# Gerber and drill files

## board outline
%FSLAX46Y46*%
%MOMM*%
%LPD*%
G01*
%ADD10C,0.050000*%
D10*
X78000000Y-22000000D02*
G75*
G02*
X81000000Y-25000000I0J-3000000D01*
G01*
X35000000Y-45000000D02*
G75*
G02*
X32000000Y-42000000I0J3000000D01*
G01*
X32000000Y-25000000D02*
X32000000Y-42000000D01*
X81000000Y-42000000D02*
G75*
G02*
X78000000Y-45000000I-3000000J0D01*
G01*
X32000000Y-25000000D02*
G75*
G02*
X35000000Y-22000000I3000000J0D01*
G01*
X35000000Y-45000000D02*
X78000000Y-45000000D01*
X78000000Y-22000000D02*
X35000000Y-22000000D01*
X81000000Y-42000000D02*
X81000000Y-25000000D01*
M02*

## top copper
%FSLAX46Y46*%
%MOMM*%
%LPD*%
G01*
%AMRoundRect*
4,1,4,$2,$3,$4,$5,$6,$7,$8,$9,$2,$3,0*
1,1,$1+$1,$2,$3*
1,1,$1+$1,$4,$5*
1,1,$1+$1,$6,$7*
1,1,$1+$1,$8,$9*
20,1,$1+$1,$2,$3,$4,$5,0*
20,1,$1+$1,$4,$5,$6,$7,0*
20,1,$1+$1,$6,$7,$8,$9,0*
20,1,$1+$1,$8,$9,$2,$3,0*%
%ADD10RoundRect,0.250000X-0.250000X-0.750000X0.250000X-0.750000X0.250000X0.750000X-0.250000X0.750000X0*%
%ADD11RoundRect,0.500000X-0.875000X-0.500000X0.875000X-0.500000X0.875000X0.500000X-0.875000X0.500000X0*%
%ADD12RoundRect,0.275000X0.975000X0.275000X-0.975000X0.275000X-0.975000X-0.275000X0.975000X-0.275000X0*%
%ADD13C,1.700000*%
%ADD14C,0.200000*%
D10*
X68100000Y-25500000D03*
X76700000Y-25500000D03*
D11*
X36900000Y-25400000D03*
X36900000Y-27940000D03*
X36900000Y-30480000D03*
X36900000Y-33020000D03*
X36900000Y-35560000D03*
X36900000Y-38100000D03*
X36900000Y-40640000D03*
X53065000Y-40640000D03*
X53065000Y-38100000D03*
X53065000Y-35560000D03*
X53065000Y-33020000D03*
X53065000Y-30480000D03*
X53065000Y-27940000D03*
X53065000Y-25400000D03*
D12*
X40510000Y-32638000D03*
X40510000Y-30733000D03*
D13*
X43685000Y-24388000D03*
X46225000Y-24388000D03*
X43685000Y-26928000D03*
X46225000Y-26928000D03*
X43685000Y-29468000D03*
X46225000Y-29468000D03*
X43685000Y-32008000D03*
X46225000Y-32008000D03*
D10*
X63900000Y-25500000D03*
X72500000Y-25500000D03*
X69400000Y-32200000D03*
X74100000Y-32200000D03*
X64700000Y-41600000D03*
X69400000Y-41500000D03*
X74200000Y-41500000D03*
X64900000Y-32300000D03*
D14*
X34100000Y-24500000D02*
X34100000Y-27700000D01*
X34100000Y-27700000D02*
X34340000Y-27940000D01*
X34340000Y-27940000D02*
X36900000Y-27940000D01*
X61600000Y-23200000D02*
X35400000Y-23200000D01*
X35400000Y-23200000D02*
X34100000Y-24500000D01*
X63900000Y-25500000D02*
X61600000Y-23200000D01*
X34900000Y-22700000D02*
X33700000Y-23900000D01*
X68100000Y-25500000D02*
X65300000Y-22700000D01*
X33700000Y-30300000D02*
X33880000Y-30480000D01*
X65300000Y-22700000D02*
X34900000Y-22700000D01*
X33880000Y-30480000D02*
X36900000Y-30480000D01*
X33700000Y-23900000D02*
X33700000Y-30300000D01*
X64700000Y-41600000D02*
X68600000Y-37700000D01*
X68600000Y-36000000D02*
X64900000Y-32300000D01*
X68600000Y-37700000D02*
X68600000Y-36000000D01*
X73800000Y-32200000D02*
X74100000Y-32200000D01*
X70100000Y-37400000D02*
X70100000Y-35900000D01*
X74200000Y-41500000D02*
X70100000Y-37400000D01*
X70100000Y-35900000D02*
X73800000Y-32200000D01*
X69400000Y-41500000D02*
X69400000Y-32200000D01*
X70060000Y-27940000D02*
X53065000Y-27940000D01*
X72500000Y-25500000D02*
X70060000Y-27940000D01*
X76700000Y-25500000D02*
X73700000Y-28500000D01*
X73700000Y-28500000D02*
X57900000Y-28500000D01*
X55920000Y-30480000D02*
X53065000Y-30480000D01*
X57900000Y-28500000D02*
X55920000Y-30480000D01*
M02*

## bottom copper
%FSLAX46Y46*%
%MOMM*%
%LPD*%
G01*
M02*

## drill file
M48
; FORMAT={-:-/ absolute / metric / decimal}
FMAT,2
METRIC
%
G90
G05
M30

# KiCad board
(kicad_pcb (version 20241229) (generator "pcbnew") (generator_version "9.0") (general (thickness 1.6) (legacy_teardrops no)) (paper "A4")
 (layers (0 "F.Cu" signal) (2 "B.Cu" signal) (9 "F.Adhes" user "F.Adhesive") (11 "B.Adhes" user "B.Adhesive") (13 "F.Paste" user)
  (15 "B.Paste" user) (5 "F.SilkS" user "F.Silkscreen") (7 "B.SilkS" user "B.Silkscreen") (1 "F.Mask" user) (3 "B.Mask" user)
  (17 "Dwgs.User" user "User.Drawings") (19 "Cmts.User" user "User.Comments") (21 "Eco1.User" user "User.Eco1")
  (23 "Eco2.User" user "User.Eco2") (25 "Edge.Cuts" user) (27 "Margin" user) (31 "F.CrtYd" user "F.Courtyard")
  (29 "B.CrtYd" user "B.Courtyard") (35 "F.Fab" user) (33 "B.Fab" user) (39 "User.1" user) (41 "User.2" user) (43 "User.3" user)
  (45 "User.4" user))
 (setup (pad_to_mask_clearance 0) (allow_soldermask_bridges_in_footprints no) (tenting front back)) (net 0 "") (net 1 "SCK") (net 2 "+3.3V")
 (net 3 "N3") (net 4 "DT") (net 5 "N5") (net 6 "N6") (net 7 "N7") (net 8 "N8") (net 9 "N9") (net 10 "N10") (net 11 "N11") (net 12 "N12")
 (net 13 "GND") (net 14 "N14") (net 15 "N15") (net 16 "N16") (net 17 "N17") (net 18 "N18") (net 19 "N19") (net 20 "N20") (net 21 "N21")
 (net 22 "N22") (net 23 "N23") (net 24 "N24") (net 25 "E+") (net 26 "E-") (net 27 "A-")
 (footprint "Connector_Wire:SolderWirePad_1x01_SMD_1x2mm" (layer "F.Cu") (at 68.1 25.5)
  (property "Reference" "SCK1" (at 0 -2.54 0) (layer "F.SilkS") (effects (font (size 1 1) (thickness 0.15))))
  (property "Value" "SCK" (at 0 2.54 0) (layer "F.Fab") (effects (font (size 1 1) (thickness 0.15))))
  (pad "1" smd roundrect (at 0 0) (size 1 2) (layers "F.Cu" "F.Mask" "F.Paste") (roundrect_rratio 0.25) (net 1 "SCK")))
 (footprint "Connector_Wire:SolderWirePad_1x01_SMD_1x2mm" (layer "F.Cu") (at 76.7 25.5)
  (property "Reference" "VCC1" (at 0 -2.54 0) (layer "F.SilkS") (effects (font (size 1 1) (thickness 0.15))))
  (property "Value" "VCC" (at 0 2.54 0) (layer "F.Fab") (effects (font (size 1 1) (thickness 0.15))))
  (pad "1" smd roundrect (at 0 0) (size 1 2) (layers "F.Cu" "F.Mask" "F.Paste") (roundrect_rratio 0.25) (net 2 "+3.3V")))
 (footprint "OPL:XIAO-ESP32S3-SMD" (layer "F.Cu") (at 44.961364 32.973)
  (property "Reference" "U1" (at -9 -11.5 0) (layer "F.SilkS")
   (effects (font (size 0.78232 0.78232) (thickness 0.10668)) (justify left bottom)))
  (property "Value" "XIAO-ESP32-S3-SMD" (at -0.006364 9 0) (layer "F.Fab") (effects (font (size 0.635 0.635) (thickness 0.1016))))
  (pad "1" smd roundrect (at -8.061364 -7.573) (size 2.75 2) (layers "F.Cu" "F.Mask" "F.Paste") (roundrect_rratio 0.25) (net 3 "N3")
   (solder_mask_margin 0.0508) (thermal_bridge_angle 45))
  (pad "2" smd roundrect (at -8.061364 -5.033) (size 2.75 2) (layers "F.Cu" "F.Mask" "F.Paste") (roundrect_rratio 0.25) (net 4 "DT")
   (solder_mask_margin 0.0508) (thermal_bridge_angle 45))
  (pad "3" smd roundrect (at -8.061364 -2.493) (size 2.75 2) (layers "F.Cu" "F.Mask" "F.Paste") (roundrect_rratio 0.25) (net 1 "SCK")
   (solder_mask_margin 0.0508) (thermal_bridge_angle 45))
  (pad "4" smd roundrect (at -8.061364 0.047) (size 2.75 2) (layers "F.Cu" "F.Mask" "F.Paste") (roundrect_rratio 0.25) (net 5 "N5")
   (solder_mask_margin 0.0508) (thermal_bridge_angle 45))
  (pad "5" smd roundrect (at -8.061364 2.587) (size 2.75 2) (layers "F.Cu" "F.Mask" "F.Paste") (roundrect_rratio 0.25) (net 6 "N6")
   (solder_mask_margin 0.0508) (thermal_bridge_angle 45))
  (pad "6" smd roundrect (at -8.061364 5.127) (size 2.75 2) (layers "F.Cu" "F.Mask" "F.Paste") (roundrect_rratio 0.25) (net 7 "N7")
   (solder_mask_margin 0.0508) (thermal_bridge_angle 45))
  (pad "7" smd roundrect (at -8.061364 7.667) (size 2.75 2) (layers "F.Cu" "F.Mask" "F.Paste") (roundrect_rratio 0.25) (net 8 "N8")
   (solder_mask_margin 0.0508) (thermal_bridge_angle 45))
  (pad "8" smd roundrect (at 8.103636 7.667) (size 2.75 2) (layers "F.Cu" "F.Mask" "F.Paste") (roundrect_rratio 0.25) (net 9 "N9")
   (solder_mask_margin 0.0508) (thermal_bridge_angle 45))
  (pad "9" smd roundrect (at 8.103636 5.127) (size 2.75 2) (layers "F.Cu" "F.Mask" "F.Paste") (roundrect_rratio 0.25) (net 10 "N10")
   (solder_mask_margin 0.0508) (thermal_bridge_angle 45))
  (pad "10" smd roundrect (at 8.103636 2.587) (size 2.75 2) (layers "F.Cu" "F.Mask" "F.Paste") (roundrect_rratio 0.25) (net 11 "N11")
   (solder_mask_margin 0.0508) (thermal_bridge_angle 45))
  (pad "11" smd roundrect (at 8.103636 0.047) (size 2.75 2) (layers "F.Cu" "F.Mask" "F.Paste") (roundrect_rratio 0.25) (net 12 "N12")
   (solder_mask_margin 0.0508) (thermal_bridge_angle 45))
  (pad "12" smd roundrect (at 8.103636 -2.493) (size 2.75 2) (layers "F.Cu" "F.Mask" "F.Paste") (roundrect_rratio 0.25) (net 2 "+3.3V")
   (solder_mask_margin 0.0508) (thermal_bridge_angle 45))
  (pad "13" smd roundrect (at 8.103636 -5.033) (size 2.75 2) (layers "F.Cu" "F.Mask" "F.Paste") (roundrect_rratio 0.25) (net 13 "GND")
   (solder_mask_margin 0.0508) (thermal_bridge_angle 45))
  (pad "14" smd roundrect (at 8.103636 -7.573) (size 2.75 2) (layers "F.Cu" "F.Mask" "F.Paste") (roundrect_rratio 0.25) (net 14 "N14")
   (solder_mask_margin 0.0508) (thermal_bridge_angle 45))
  (pad "15" smd roundrect (at -4.451364 -0.335 180) (size 2.5 1.1) (layers "F.Cu" "F.Mask" "F.Paste") (roundrect_rratio 0.25) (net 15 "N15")
   (solder_mask_margin 0.0508) (thermal_bridge_angle 45))
  (pad "16" smd roundrect (at -4.451364 -2.24 180) (size 2.5 1.1) (layers "F.Cu" "F.Mask" "F.Paste") (roundrect_rratio 0.25) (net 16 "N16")
   (solder_mask_margin 0.0508) (thermal_bridge_angle 45))
  (pad "17" smd circle (at -1.276364 -8.585) (size 1.7 1.7) (layers "F.Cu" "F.Mask" "F.Paste") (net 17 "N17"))
  (pad "18" smd circle (at 1.263636 -8.585) (size 1.7 1.7) (layers "F.Cu" "F.Mask" "F.Paste") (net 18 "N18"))
  (pad "19" smd circle (at -1.276364 -6.045) (size 1.7 1.7) (layers "F.Cu" "F.Mask" "F.Paste") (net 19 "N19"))
  (pad "20" smd circle (at 1.263636 -6.045) (size 1.7 1.7) (layers "F.Cu" "F.Mask" "F.Paste") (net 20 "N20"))
  (pad "21" smd circle (at -1.276364 -3.505) (size 1.7 1.7) (layers "F.Cu" "F.Mask" "F.Paste") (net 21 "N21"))
  (pad "22" smd circle (at 1.263636 -3.505) (size 1.7 1.7) (layers "F.Cu" "F.Mask" "F.Paste") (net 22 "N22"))
  (pad "23" smd circle (at -1.276364 -0.965) (size 1.7 1.7) (layers "F.Cu" "F.Mask" "F.Paste") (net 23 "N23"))
  (pad "24" smd circle (at 1.263636 -0.965) (size 1.7 1.7) (layers "F.Cu" "F.Mask" "F.Paste") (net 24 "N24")))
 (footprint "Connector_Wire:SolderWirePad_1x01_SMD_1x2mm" (layer "F.Cu") (at 63.9 25.5)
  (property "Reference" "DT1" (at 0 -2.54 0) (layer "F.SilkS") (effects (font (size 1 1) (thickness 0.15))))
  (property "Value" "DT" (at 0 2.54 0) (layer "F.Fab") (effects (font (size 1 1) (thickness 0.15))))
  (pad "1" smd roundrect (at 0 0) (size 1 2) (layers "F.Cu" "F.Mask" "F.Paste") (roundrect_rratio 0.25) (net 4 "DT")))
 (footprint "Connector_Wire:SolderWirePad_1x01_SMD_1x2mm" (layer "F.Cu") (at 72.5 25.5)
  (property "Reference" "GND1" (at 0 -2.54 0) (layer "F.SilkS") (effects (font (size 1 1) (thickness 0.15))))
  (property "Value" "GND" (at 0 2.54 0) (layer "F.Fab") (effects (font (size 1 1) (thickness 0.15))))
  (pad "1" smd roundrect (at 0 0) (size 1 2) (layers "F.Cu" "F.Mask" "F.Paste") (roundrect_rratio 0.25) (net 13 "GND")))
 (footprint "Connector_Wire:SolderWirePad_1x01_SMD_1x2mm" (layer "F.Cu") (at 69.4 32.2)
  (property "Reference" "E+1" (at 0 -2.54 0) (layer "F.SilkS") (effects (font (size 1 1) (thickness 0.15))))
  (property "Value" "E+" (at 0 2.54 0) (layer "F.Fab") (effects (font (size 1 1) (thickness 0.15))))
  (pad "1" smd roundrect (at 0 0) (size 1 2) (layers "F.Cu" "F.Mask" "F.Paste") (roundrect_rratio 0.25) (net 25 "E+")))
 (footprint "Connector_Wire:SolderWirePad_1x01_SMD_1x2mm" (layer "F.Cu") (at 74.1 32.2)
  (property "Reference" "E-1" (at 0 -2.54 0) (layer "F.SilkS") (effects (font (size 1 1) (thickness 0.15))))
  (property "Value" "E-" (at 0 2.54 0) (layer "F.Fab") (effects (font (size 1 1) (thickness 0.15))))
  (pad "1" smd roundrect (at 0 0) (size 1 2) (layers "F.Cu" "F.Mask" "F.Paste") (roundrect_rratio 0.25) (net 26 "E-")))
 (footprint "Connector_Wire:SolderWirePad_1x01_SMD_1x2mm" (layer "F.Cu") (at 64.7 41.6)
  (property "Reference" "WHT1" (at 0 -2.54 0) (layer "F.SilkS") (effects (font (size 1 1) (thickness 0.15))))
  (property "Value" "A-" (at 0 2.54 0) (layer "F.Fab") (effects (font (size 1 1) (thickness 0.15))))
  (pad "1" smd roundrect (at 0 0) (size 1 2) (layers "F.Cu" "F.Mask" "F.Paste") (roundrect_rratio 0.25) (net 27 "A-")))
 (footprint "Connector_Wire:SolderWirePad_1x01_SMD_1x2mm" (layer "F.Cu") (at 69.4 41.5)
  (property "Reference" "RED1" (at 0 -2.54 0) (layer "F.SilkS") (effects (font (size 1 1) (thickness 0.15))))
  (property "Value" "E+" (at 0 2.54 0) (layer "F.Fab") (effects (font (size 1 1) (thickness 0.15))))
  (pad "1" smd roundrect (at 0 0) (size 1 2) (layers "F.Cu" "F.Mask" "F.Paste") (roundrect_rratio 0.25) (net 25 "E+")))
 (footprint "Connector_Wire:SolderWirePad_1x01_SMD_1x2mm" (layer "F.Cu") (at 74.2 41.5)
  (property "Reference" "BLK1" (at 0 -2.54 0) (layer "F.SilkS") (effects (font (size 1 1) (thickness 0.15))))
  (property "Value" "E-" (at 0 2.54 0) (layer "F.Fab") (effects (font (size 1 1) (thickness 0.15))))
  (pad "1" smd roundrect (at 0 0) (size 1 2) (layers "F.Cu" "F.Mask" "F.Paste") (roundrect_rratio 0.25) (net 26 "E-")))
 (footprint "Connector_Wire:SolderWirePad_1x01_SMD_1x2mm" (layer "F.Cu") (at 64.9 32.3)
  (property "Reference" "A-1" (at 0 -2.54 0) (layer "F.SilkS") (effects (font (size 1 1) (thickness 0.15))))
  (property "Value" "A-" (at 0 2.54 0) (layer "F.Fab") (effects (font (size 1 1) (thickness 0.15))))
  (pad "1" smd roundrect (at 0 0) (size 1 2) (layers "F.Cu" "F.Mask" "F.Paste") (roundrect_rratio 0.25) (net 27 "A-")))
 (gr_arc (start 78 22) (mid 80.12132 22.87868) (end 81 25) (stroke (width 0.05) (type default)) (layer "Edge.Cuts"))
 (gr_arc (start 35 45) (mid 32.87868 44.12132) (end 32 42) (stroke (width 0.05) (type default)) (layer "Edge.Cuts"))
 (gr_line (start 32 25) (end 32 42) (stroke (width 0.05) (type default)) (layer "Edge.Cuts"))
 (gr_arc (start 81 42) (mid 80.12132 44.12132) (end 78 45) (stroke (width 0.05) (type default)) (layer "Edge.Cuts"))
 (gr_arc (start 32 25) (mid 32.87868 22.87868) (end 35 22) (stroke (width 0.05) (type default)) (layer "Edge.Cuts"))
 (gr_line (start 35 45) (end 78 45) (stroke (width 0.05) (type default)) (layer "Edge.Cuts"))
 (gr_line (start 78 22) (end 35 22) (stroke (width 0.05) (type default)) (layer "Edge.Cuts"))
 (gr_line (start 81 42) (end 81 25) (stroke (width 0.05) (type default)) (layer "Edge.Cuts"))
 (segment (start 34.1 24.5) (end 34.1 27.7) (width 0.2) (layer "F.Cu") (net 4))
 (segment (start 34.1 27.7) (end 34.34 27.94) (width 0.2) (layer "F.Cu") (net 4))
 (segment (start 34.34 27.94) (end 36.9 27.94) (width 0.2) (layer "F.Cu") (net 4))
 (segment (start 61.6 23.2) (end 35.4 23.2) (width 0.2) (layer "F.Cu") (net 4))
 (segment (start 35.4 23.2) (end 34.1 24.5) (width 0.2) (layer "F.Cu") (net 4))
 (segment (start 63.9 25.5) (end 61.6 23.2) (width 0.2) (layer "F.Cu") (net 4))
 (segment (start 34.9 22.7) (end 33.7 23.9) (width 0.2) (layer "F.Cu") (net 1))
 (segment (start 68.1 25.5) (end 65.3 22.7) (width 0.2) (layer "F.Cu") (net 1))
 (segment (start 33.7 30.3) (end 33.88 30.48) (width 0.2) (layer "F.Cu") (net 1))
 (segment (start 65.3 22.7) (end 34.9 22.7) (width 0.2) (layer "F.Cu") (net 1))
 (segment (start 33.88 30.48) (end 36.9 30.48) (width 0.2) (layer "F.Cu") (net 1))
 (segment (start 33.7 23.9) (end 33.7 30.3) (width 0.2) (layer "F.Cu") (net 1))
 (segment (start 64.7 41.6) (end 68.6 37.7) (width 0.2) (layer "F.Cu") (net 27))
 (segment (start 68.6 36) (end 64.9 32.3) (width 0.2) (layer "F.Cu") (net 27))
 (segment (start 68.6 37.7) (end 68.6 36) (width 0.2) (layer "F.Cu") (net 27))
 (segment (start 73.8 32.2) (end 74.1 32.2) (width 0.2) (layer "F.Cu") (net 26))
 (segment (start 70.1 37.4) (end 70.1 35.9) (width 0.2) (layer "F.Cu") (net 26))
 (segment (start 74.2 41.5) (end 70.1 37.4) (width 0.2) (layer "F.Cu") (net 26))
 (segment (start 70.1 35.9) (end 73.8 32.2) (width 0.2) (layer "F.Cu") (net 26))
 (segment (start 69.4 41.5) (end 69.4 32.2) (width 0.2) (layer "F.Cu") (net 25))
 (segment (start 70.06 27.94) (end 53.065 27.94) (width 0.2) (layer "F.Cu") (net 13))
 (segment (start 72.5 25.5) (end 70.06 27.94) (width 0.2) (layer "F.Cu") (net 13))
 (segment (start 76.7 25.5) (end 73.7 28.5) (width 0.2) (layer "F.Cu") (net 2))
 (segment (start 73.7 28.5) (end 57.9 28.5) (width 0.2) (layer "F.Cu") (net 2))
 (segment (start 55.92 30.48) (end 53.065 30.48) (width 0.2) (layer "F.Cu") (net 2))
 (segment (start 57.9 28.5) (end 55.92 30.48) (width 0.2) (layer "F.Cu") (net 2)))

